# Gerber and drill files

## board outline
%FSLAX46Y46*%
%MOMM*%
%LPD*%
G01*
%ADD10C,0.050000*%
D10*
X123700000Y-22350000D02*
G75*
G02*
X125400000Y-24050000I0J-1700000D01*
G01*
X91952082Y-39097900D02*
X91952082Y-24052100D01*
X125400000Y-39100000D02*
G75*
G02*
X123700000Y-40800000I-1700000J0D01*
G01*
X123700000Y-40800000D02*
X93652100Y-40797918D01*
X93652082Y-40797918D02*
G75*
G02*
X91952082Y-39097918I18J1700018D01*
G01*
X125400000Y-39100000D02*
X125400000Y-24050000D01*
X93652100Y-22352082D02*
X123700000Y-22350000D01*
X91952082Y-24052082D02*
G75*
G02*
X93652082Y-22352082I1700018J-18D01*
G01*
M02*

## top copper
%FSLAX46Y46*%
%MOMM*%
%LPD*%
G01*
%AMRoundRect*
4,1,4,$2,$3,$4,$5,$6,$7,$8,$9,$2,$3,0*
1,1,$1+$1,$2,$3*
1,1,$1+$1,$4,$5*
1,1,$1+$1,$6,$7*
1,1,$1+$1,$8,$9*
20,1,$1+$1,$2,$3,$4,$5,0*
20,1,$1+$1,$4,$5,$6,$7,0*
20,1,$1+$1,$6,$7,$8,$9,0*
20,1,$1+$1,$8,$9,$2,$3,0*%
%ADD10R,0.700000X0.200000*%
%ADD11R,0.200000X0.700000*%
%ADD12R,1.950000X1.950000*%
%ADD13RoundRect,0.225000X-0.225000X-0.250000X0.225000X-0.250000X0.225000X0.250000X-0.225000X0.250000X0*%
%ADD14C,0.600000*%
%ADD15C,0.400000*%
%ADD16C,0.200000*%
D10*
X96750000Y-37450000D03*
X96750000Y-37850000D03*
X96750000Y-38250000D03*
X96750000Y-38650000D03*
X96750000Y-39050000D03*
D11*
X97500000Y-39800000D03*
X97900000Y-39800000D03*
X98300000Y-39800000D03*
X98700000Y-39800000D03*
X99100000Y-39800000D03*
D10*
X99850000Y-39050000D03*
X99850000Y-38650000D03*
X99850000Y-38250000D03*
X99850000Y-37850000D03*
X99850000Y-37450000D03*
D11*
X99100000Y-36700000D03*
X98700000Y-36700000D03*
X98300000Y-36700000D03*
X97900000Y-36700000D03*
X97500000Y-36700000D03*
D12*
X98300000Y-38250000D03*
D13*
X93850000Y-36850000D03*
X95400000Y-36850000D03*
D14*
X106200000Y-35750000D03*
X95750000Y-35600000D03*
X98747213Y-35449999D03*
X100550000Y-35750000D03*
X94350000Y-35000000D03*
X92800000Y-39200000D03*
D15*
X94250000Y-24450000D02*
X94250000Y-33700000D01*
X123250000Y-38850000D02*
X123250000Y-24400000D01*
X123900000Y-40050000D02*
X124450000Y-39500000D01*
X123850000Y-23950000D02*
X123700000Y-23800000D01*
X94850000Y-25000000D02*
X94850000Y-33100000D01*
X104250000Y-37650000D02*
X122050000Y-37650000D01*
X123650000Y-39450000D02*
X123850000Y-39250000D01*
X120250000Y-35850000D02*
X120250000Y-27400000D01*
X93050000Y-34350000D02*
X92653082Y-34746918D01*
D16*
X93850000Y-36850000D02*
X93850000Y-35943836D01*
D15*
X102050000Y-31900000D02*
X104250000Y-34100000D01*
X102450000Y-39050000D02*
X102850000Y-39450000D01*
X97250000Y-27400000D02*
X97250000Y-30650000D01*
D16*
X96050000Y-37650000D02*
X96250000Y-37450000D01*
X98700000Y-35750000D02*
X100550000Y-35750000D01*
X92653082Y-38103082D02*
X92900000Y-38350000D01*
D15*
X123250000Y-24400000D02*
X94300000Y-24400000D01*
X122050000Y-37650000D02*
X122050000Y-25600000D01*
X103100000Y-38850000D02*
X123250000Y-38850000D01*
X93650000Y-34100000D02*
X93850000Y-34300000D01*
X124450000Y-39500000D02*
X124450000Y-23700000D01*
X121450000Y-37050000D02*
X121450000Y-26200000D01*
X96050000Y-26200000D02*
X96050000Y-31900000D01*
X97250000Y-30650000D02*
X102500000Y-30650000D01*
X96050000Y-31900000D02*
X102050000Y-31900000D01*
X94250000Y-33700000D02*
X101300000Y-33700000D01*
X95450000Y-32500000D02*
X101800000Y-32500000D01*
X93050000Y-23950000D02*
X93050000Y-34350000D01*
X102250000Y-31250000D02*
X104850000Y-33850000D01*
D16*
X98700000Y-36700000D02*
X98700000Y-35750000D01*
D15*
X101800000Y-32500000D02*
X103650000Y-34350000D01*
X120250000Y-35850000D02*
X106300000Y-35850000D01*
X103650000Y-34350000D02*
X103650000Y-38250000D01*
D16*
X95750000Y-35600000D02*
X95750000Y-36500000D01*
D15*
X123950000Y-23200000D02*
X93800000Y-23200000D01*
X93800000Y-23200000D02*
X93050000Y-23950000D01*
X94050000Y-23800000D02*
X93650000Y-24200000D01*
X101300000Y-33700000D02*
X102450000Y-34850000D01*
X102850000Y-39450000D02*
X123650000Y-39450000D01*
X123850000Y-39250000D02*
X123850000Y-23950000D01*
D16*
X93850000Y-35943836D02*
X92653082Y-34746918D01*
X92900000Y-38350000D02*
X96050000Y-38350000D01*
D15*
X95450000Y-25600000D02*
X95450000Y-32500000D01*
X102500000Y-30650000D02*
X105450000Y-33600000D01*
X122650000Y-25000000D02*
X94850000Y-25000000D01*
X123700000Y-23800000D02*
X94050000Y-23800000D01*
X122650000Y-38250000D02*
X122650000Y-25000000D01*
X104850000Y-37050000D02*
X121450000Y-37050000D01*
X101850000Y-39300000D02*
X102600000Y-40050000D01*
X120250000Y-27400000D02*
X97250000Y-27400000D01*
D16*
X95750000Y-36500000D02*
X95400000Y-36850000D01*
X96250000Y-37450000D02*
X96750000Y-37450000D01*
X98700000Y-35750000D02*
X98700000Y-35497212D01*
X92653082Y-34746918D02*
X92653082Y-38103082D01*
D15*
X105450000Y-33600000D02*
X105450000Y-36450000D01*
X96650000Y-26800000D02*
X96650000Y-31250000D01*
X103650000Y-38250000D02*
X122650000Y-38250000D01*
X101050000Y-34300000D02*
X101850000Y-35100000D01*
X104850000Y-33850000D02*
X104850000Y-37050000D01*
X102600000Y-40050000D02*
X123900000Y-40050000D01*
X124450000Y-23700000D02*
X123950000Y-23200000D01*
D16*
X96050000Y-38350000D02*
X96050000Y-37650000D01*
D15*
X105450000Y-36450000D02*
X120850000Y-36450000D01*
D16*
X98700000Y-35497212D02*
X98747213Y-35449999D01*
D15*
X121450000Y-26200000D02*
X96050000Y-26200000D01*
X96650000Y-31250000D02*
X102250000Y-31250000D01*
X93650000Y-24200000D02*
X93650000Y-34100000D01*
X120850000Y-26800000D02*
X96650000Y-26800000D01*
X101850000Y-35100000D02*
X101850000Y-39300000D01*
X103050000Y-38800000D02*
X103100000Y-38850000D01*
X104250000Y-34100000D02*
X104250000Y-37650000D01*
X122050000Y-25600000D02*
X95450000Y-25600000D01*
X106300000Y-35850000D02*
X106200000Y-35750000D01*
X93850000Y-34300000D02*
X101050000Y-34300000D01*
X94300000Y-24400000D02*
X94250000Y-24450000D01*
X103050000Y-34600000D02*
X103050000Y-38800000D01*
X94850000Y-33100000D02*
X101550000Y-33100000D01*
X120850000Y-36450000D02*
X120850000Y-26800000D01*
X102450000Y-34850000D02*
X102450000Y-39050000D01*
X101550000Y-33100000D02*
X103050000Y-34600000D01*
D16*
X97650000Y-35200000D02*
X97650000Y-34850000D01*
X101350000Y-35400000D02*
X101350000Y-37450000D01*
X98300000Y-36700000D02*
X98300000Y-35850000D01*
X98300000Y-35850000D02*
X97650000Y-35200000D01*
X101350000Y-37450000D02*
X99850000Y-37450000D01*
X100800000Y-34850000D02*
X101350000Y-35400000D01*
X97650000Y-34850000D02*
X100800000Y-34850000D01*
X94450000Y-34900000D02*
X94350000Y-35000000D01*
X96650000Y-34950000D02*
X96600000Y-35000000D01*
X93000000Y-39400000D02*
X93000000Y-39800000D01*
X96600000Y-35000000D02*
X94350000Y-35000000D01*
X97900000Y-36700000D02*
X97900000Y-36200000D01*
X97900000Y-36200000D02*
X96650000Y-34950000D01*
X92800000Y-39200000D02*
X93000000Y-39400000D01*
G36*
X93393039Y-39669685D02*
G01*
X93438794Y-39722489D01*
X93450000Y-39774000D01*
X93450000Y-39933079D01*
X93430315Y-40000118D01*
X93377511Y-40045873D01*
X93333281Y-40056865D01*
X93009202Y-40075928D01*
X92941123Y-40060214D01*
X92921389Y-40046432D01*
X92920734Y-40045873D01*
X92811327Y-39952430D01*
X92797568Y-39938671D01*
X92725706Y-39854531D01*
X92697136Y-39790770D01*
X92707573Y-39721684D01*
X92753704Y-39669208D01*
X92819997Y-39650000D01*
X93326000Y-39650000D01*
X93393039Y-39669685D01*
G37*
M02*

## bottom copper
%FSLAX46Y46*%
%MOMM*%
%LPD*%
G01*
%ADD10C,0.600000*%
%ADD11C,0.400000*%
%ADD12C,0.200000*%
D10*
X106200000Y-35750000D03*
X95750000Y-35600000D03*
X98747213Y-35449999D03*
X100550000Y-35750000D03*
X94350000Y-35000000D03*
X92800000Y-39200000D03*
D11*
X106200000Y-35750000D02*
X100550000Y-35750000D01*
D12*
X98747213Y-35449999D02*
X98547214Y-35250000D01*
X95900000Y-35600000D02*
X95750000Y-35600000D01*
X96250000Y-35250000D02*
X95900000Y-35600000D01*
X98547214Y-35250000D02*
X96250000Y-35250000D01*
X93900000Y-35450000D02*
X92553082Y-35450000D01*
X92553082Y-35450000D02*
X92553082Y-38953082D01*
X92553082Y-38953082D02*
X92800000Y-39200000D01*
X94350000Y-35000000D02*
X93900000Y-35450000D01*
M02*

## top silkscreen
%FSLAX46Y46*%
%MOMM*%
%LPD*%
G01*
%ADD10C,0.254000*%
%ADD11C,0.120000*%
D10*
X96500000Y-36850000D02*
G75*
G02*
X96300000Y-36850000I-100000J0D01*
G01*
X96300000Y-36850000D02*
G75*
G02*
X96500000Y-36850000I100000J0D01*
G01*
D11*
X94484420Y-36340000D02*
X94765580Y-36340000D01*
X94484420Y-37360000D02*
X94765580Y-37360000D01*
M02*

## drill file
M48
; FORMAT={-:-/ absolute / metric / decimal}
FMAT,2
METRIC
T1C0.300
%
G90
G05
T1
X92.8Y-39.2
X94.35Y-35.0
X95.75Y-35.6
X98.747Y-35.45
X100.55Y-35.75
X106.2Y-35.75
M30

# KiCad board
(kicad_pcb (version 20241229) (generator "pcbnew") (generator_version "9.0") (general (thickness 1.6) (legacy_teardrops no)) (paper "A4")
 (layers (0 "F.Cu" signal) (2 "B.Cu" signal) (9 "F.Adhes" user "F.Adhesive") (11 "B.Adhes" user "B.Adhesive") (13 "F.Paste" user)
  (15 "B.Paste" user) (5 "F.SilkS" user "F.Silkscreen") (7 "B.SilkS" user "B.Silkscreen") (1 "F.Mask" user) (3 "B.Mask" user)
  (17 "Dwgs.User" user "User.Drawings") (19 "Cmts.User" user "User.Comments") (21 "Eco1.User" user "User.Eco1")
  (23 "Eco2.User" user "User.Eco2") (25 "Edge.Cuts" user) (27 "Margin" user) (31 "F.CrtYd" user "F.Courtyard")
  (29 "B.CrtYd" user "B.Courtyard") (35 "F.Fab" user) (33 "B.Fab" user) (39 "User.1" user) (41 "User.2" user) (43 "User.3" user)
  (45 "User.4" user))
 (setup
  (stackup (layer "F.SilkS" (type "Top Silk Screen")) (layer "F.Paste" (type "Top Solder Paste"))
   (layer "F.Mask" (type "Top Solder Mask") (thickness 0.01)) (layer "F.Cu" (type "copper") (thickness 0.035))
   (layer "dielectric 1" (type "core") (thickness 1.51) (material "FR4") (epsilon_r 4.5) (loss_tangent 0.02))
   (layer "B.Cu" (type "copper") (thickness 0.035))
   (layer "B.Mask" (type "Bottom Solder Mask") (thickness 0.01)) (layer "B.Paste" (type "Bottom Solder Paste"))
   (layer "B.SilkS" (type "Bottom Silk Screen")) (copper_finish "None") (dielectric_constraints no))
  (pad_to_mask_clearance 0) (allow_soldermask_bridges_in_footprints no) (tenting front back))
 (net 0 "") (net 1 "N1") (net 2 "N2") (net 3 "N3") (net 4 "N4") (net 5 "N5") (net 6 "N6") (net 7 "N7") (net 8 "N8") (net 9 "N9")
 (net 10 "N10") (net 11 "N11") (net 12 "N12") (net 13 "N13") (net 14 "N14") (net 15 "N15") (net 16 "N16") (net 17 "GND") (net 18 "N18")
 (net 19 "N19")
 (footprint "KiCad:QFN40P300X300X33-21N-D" (layer "F.Cu") (at 98.3 38.25)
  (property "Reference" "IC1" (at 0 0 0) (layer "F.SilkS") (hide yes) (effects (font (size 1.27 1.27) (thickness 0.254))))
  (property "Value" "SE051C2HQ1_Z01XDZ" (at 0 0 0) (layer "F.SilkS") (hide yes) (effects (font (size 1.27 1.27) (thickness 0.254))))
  (fp_circle (center -1.9 -1.4) (end -1.8 -1.4) (stroke (width 0.254) (type solid)) (fill no) (layer "F.SilkS"))
  (pad "1" smd rect (at -1.55 -0.8 90) (size 0.2 0.7) (layers "F.Cu" "F.Mask" "F.Paste") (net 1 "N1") (solder_mask_margin 0.04)
   (thermal_bridge_angle 45))
  (pad "2" smd rect (at -1.55 -0.4 90) (size 0.2 0.7) (layers "F.Cu" "F.Mask" "F.Paste") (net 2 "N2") (solder_mask_margin 0.04)
   (thermal_bridge_angle 45))
  (pad "3" smd rect (at -1.55 0 90) (size 0.2 0.7) (layers "F.Cu" "F.Mask" "F.Paste") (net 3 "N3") (solder_mask_margin 0.04)
   (thermal_bridge_angle 45))
  (pad "4" smd rect (at -1.55 0.4 90) (size 0.2 0.7) (layers "F.Cu" "F.Mask" "F.Paste") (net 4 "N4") (solder_mask_margin 0.04)
   (thermal_bridge_angle 45))
  (pad "5" smd rect (at -1.55 0.8 90) (size 0.2 0.7) (layers "F.Cu" "F.Mask" "F.Paste") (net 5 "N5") (solder_mask_margin 0.04)
   (thermal_bridge_angle 45))
  (pad "6" smd rect (at -0.8 1.55) (size 0.2 0.7) (layers "F.Cu" "F.Mask" "F.Paste") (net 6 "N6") (solder_mask_margin 0.04)
   (thermal_bridge_angle 45))
  (pad "7" smd rect (at -0.4 1.55) (size 0.2 0.7) (layers "F.Cu" "F.Mask" "F.Paste") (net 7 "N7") (solder_mask_margin 0.04)
   (thermal_bridge_angle 45))
  (pad "8" smd rect (at 0 1.55) (size 0.2 0.7) (layers "F.Cu" "F.Mask" "F.Paste") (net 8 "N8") (solder_mask_margin 0.04)
   (thermal_bridge_angle 45))
  (pad "9" smd rect (at 0.4 1.55) (size 0.2 0.7) (layers "F.Cu" "F.Mask" "F.Paste") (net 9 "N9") (solder_mask_margin 0.04)
   (thermal_bridge_angle 45))
  (pad "10" smd rect (at 0.8 1.55) (size 0.2 0.7) (layers "F.Cu" "F.Mask" "F.Paste") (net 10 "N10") (solder_mask_margin 0.04)
   (thermal_bridge_angle 45))
  (pad "11" smd rect (at 1.55 0.8 90) (size 0.2 0.7) (layers "F.Cu" "F.Mask" "F.Paste") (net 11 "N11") (solder_mask_margin 0.04)
   (thermal_bridge_angle 45))
  (pad "12" smd rect (at 1.55 0.4 90) (size 0.2 0.7) (layers "F.Cu" "F.Mask" "F.Paste") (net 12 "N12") (solder_mask_margin 0.04)
   (thermal_bridge_angle 45))
  (pad "13" smd rect (at 1.55 0 90) (size 0.2 0.7) (layers "F.Cu" "F.Mask" "F.Paste") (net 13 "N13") (solder_mask_margin 0.04)
   (thermal_bridge_angle 45))
  (pad "14" smd rect (at 1.55 -0.4 90) (size 0.2 0.7) (layers "F.Cu" "F.Mask" "F.Paste") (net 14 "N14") (solder_mask_margin 0.04)
   (thermal_bridge_angle 45))
  (pad "15" smd rect (at 1.55 -0.8 90) (size 0.2 0.7) (layers "F.Cu" "F.Mask" "F.Paste") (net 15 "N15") (solder_mask_margin 0.04)
   (thermal_bridge_angle 45))
  (pad "16" smd rect (at 0.8 -1.55) (size 0.2 0.7) (layers "F.Cu" "F.Mask" "F.Paste") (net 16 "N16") (solder_mask_margin 0.04)
   (thermal_bridge_angle 45))
  (pad "17" smd rect (at 0.4 -1.55) (size 0.2 0.7) (layers "F.Cu" "F.Mask" "F.Paste") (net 1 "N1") (solder_mask_margin 0.04)
   (thermal_bridge_angle 45))
  (pad "18" smd rect (at 0 -1.55) (size 0.2 0.7) (layers "F.Cu" "F.Mask" "F.Paste") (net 15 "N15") (solder_mask_margin 0.04)
   (thermal_bridge_angle 45))
  (pad "19" smd rect (at -0.4 -1.55) (size 0.2 0.7) (layers "F.Cu" "F.Mask" "F.Paste") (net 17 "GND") (solder_mask_margin 0.04)
   (thermal_bridge_angle 45))
  (pad "20" smd rect (at -0.8 -1.55) (size 0.2 0.7) (layers "F.Cu" "F.Mask" "F.Paste") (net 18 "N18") (solder_mask_margin 0.04)
   (thermal_bridge_angle 45))
  (pad "21" smd rect (at 0 0) (size 1.95 1.95) (layers "F.Cu" "F.Mask" "F.Paste") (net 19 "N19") (thermal_bridge_angle 45)))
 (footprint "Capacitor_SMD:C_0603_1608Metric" (layer "F.Cu") (at 94.625 36.85)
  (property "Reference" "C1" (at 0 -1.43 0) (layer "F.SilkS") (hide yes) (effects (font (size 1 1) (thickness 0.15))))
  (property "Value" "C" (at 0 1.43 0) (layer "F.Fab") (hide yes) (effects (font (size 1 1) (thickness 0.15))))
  (fp_line (start -0.14058 -0.51) (end 0.14058 -0.51) (stroke (width 0.12) (type solid)) (layer "F.SilkS"))
  (fp_line (start -0.14058 0.51) (end 0.14058 0.51) (stroke (width 0.12) (type solid)) (layer "F.SilkS"))
  (pad "1" smd roundrect (at -0.775 0) (size 0.9 0.95) (layers "F.Cu" "F.Mask" "F.Paste") (roundrect_rratio 0.25) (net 1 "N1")
   (solder_mask_margin 0.04))
  (pad "2" smd roundrect (at 0.775 0) (size 0.9 0.95) (layers "F.Cu" "F.Mask" "F.Paste") (roundrect_rratio 0.25) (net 1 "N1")
   (solder_mask_margin 0.04)))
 (gr_arc (start 123.7 22.35) (mid 124.902082 22.847918) (end 125.4 24.05) (stroke (width 0.05) (type default)) (layer "Edge.Cuts"))
 (gr_line (start 91.952082 39.0979) (end 91.952082 24.0521) (stroke (width 0.05) (type default)) (layer "Edge.Cuts"))
 (gr_arc (start 125.4 39.1) (mid 124.902082 40.302082) (end 123.7 40.8) (stroke (width 0.05) (type default)) (layer "Edge.Cuts"))
 (gr_line (start 123.7 40.8) (end 93.6521 40.797918) (stroke (width 0.05) (type default)) (layer "Edge.Cuts"))
 (gr_arc (start 93.652082 40.797918) (mid 92.45 40.3) (end 91.952082 39.097918) (stroke (width 0.05) (type default)) (layer "Edge.Cuts"))
 (gr_line (start 125.4 39.1) (end 125.4 24.05) (stroke (width 0.05) (type default)) (layer "Edge.Cuts"))
 (gr_line (start 93.6521 22.352082) (end 123.7 22.35) (stroke (width 0.05) (type default)) (layer "Edge.Cuts"))
 (gr_arc (start 91.952082 24.052082) (mid 92.45 22.85) (end 93.652082 22.352082) (stroke (width 0.05) (type default)) (layer "Edge.Cuts"))
 (segment (start 94.25 24.45) (end 94.25 33.7) (width 0.4) (layer "F.Cu") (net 1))
 (segment (start 123.25 38.85) (end 123.25 24.4) (width 0.4) (layer "F.Cu") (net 1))
 (segment (start 123.9 40.05) (end 124.45 39.5) (width 0.4) (layer "F.Cu") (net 1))
 (segment (start 123.85 23.95) (end 123.7 23.8) (width 0.4) (layer "F.Cu") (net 1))
 (segment (start 94.85 25) (end 94.85 33.1) (width 0.4) (layer "F.Cu") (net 1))
 (segment (start 104.25 37.65) (end 122.05 37.65) (width 0.4) (layer "F.Cu") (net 1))
 (segment (start 123.65 39.45) (end 123.85 39.25) (width 0.4) (layer "F.Cu") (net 1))
 (segment (start 120.25 35.85) (end 120.25 27.4) (width 0.4) (layer "F.Cu") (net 1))
 (segment (start 93.05 34.35) (end 92.653082 34.746918) (width 0.4) (layer "F.Cu") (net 1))
 (segment (start 93.85 36.85) (end 93.85 35.943836) (width 0.2) (layer "F.Cu") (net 1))
 (segment (start 102.05 31.9) (end 104.25 34.1) (width 0.4) (layer "F.Cu") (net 1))
 (segment (start 102.45 39.05) (end 102.85 39.45) (width 0.4) (layer "F.Cu") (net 1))
 (segment (start 97.25 27.4) (end 97.25 30.65) (width 0.4) (layer "F.Cu") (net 1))
 (segment (start 96.05 37.65) (end 96.25 37.45) (width 0.2) (layer "F.Cu") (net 1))
 (segment (start 98.7 35.75) (end 100.55 35.75) (width 0.2) (layer "F.Cu") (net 1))
 (segment (start 92.653082 38.103082) (end 92.9 38.35) (width 0.2) (layer "F.Cu") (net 1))
 (segment (start 123.25 24.4) (end 94.3 24.4) (width 0.4) (layer "F.Cu") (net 1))
 (segment (start 122.05 37.65) (end 122.05 25.6) (width 0.4) (layer "F.Cu") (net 1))
 (segment (start 103.1 38.85) (end 123.25 38.85) (width 0.4) (layer "F.Cu") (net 1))
 (segment (start 93.65 34.1) (end 93.85 34.3) (width 0.4) (layer "F.Cu") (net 1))
 (segment (start 124.45 39.5) (end 124.45 23.7) (width 0.4) (layer "F.Cu") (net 1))
 (segment (start 121.45 37.05) (end 121.45 26.2) (width 0.4) (layer "F.Cu") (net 1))
 (segment (start 96.05 26.2) (end 96.05 31.9) (width 0.4) (layer "F.Cu") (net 1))
 (segment (start 97.25 30.65) (end 102.5 30.65) (width 0.4) (layer "F.Cu") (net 1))
 (segment (start 96.05 31.9) (end 102.05 31.9) (width 0.4) (layer "F.Cu") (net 1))
 (segment (start 94.25 33.7) (end 101.3 33.7) (width 0.4) (layer "F.Cu") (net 1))
 (segment (start 95.45 32.5) (end 101.8 32.5) (width 0.4) (layer "F.Cu") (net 1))
 (segment (start 93.05 23.95) (end 93.05 34.35) (width 0.4) (layer "F.Cu") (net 1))
 (segment (start 102.25 31.25) (end 104.85 33.85) (width 0.4) (layer "F.Cu") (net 1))
 (segment (start 98.7 36.7) (end 98.7 35.75) (width 0.2) (layer "F.Cu") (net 1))
 (segment (start 101.8 32.5) (end 103.65 34.35) (width 0.4) (layer "F.Cu") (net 1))
 (segment (start 120.25 35.85) (end 106.3 35.85) (width 0.4) (layer "F.Cu") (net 1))
 (segment (start 103.65 34.35) (end 103.65 38.25) (width 0.4) (layer "F.Cu") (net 1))
 (segment (start 95.75 35.6) (end 95.75 36.5) (width 0.2) (layer "F.Cu") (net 1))
 (segment (start 123.95 23.2) (end 93.8 23.2) (width 0.4) (layer "F.Cu") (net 1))
 (segment (start 93.8 23.2) (end 93.05 23.95) (width 0.4) (layer "F.Cu") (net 1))
 (segment (start 94.05 23.8) (end 93.65 24.2) (width 0.4) (layer "F.Cu") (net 1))
 (segment (start 101.3 33.7) (end 102.45 34.85) (width 0.4) (layer "F.Cu") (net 1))
 (segment (start 102.85 39.45) (end 123.65 39.45) (width 0.4) (layer "F.Cu") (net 1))
 (segment (start 123.85 39.25) (end 123.85 23.95) (width 0.4) (layer "F.Cu") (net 1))
 (segment (start 93.85 35.943836) (end 92.653082 34.746918) (width 0.2) (layer "F.Cu") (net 1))
 (segment (start 92.9 38.35) (end 96.05 38.35) (width 0.2) (layer "F.Cu") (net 1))
 (segment (start 95.45 25.6) (end 95.45 32.5) (width 0.4) (layer "F.Cu") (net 1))
 (segment (start 102.5 30.65) (end 105.45 33.6) (width 0.4) (layer "F.Cu") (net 1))
 (segment (start 122.65 25) (end 94.85 25) (width 0.4) (layer "F.Cu") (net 1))
 (segment (start 123.7 23.8) (end 94.05 23.8) (width 0.4) (layer "F.Cu") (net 1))
 (segment (start 122.65 38.25) (end 122.65 25) (width 0.4) (layer "F.Cu") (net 1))
 (segment (start 104.85 37.05) (end 121.45 37.05) (width 0.4) (layer "F.Cu") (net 1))
 (segment (start 101.85 39.3) (end 102.6 40.05) (width 0.4) (layer "F.Cu") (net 1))
 (segment (start 120.25 27.4) (end 97.25 27.4) (width 0.4) (layer "F.Cu") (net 1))
 (segment (start 95.75 36.5) (end 95.4 36.85) (width 0.2) (layer "F.Cu") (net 1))
 (segment (start 96.25 37.45) (end 96.75 37.45) (width 0.2) (layer "F.Cu") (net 1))
 (segment (start 98.7 35.75) (end 98.7 35.497212) (width 0.2) (layer "F.Cu") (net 1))
 (segment (start 92.653082 34.746918) (end 92.653082 38.103082) (width 0.2) (layer "F.Cu") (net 1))
 (segment (start 105.45 33.6) (end 105.45 36.45) (width 0.4) (layer "F.Cu") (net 1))
 (segment (start 96.65 26.8) (end 96.65 31.25) (width 0.4) (layer "F.Cu") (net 1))
 (segment (start 103.65 38.25) (end 122.65 38.25) (width 0.4) (layer "F.Cu") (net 1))
 (segment (start 101.05 34.3) (end 101.85 35.1) (width 0.4) (layer "F.Cu") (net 1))
 (segment (start 104.85 33.85) (end 104.85 37.05) (width 0.4) (layer "F.Cu") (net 1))
 (segment (start 102.6 40.05) (end 123.9 40.05) (width 0.4) (layer "F.Cu") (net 1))
 (segment (start 124.45 23.7) (end 123.95 23.2) (width 0.4) (layer "F.Cu") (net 1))
 (segment (start 96.05 38.35) (end 96.05 37.65) (width 0.2) (layer "F.Cu") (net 1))
 (segment (start 105.45 36.45) (end 120.85 36.45) (width 0.4) (layer "F.Cu") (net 1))
 (segment (start 98.7 35.497212) (end 98.747213 35.449999) (width 0.2) (layer "F.Cu") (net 1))
 (segment (start 121.45 26.2) (end 96.05 26.2) (width 0.4) (layer "F.Cu") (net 1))
 (segment (start 96.65 31.25) (end 102.25 31.25) (width 0.4) (layer "F.Cu") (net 1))
 (segment (start 93.65 24.2) (end 93.65 34.1) (width 0.4) (layer "F.Cu") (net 1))
 (segment (start 120.85 26.8) (end 96.65 26.8) (width 0.4) (layer "F.Cu") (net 1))
 (segment (start 101.85 35.1) (end 101.85 39.3) (width 0.4) (layer "F.Cu") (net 1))
 (segment (start 103.05 38.8) (end 103.1 38.85) (width 0.4) (layer "F.Cu") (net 1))
 (segment (start 104.25 34.1) (end 104.25 37.65) (width 0.4) (layer "F.Cu") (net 1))
 (segment (start 122.05 25.6) (end 95.45 25.6) (width 0.4) (layer "F.Cu") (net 1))
 (segment (start 106.3 35.85) (end 106.2 35.75) (width 0.4) (layer "F.Cu") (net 1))
 (segment (start 93.85 34.3) (end 101.05 34.3) (width 0.4) (layer "F.Cu") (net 1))
 (segment (start 94.3 24.4) (end 94.25 24.45) (width 0.4) (layer "F.Cu") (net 1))
 (segment (start 103.05 34.6) (end 103.05 38.8) (width 0.4) (layer "F.Cu") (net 1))
 (segment (start 94.85 33.1) (end 101.55 33.1) (width 0.4) (layer "F.Cu") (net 1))
 (segment (start 120.85 36.45) (end 120.85 26.8) (width 0.4) (layer "F.Cu") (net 1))
 (segment (start 102.45 34.85) (end 102.45 39.05) (width 0.4) (layer "F.Cu") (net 1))
 (segment (start 101.55 33.1) (end 103.05 34.6) (width 0.4) (layer "F.Cu") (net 1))
 (via (at 106.2 35.75) (size 0.6) (drill 0.3) (layers "F.Cu" "B.Cu") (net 1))
 (via (at 95.75 35.6) (size 0.6) (drill 0.3) (layers "F.Cu" "B.Cu") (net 1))
 (via (at 98.747213 35.449999) (size 0.6) (drill 0.3) (layers "F.Cu" "B.Cu") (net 1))
 (via (at 100.55 35.75) (size 0.6) (drill 0.3) (layers "F.Cu" "B.Cu") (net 1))
 (segment (start 106.2 35.75) (end 100.55 35.75) (width 0.4) (layer "B.Cu") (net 1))
 (segment (start 98.747213 35.449999) (end 98.547214 35.25) (width 0.2) (layer "B.Cu") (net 1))
 (segment (start 95.9 35.6) (end 95.75 35.6) (width 0.2) (layer "B.Cu") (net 1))
 (segment (start 96.25 35.25) (end 95.9 35.6) (width 0.2) (layer "B.Cu") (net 1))
 (segment (start 98.547214 35.25) (end 96.25 35.25) (width 0.2) (layer "B.Cu") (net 1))
 (segment (start 97.65 35.2) (end 97.65 34.85) (width 0.2) (layer "F.Cu") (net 15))
 (segment (start 101.35 35.4) (end 101.35 37.45) (width 0.2) (layer "F.Cu") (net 15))
 (segment (start 98.3 36.7) (end 98.3 35.85) (width 0.2) (layer "F.Cu") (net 15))
 (segment (start 98.3 35.85) (end 97.65 35.2) (width 0.2) (layer "F.Cu") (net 15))
 (segment (start 101.35 37.45) (end 99.85 37.45) (width 0.2) (layer "F.Cu") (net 15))
 (segment (start 100.8 34.85) (end 101.35 35.4) (width 0.2) (layer "F.Cu") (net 15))
 (segment (start 97.65 34.85) (end 100.8 34.85) (width 0.2) (layer "F.Cu") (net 15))
 (segment (start 94.45 34.9) (end 94.35 35) (width 0.2) (layer "F.Cu") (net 17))
 (segment (start 96.65 34.95) (end 96.6 35) (width 0.2) (layer "F.Cu") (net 17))
 (segment (start 93 39.4) (end 93 39.8) (width 0.2) (layer "F.Cu") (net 17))
 (segment (start 96.6 35) (end 94.35 35) (width 0.2) (layer "F.Cu") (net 17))
 (segment (start 97.9 36.7) (end 97.9 36.2) (width 0.2) (layer "F.Cu") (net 17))
 (segment (start 97.9 36.2) (end 96.65 34.95) (width 0.2) (layer "F.Cu") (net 17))
 (segment (start 92.8 39.2) (end 93 39.4) (width 0.2) (layer "F.Cu") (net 17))
 (via (at 94.35 35) (size 0.6) (drill 0.3) (layers "F.Cu" "B.Cu") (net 17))
 (via (at 92.8 39.2) (size 0.6) (drill 0.3) (layers "F.Cu" "B.Cu") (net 17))
 (segment (start 93.9 35.45) (end 92.553082 35.45) (width 0.2) (layer "B.Cu") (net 17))
 (segment (start 92.553082 35.45) (end 92.553082 38.953082) (width 0.2) (layer "B.Cu") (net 17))
 (segment (start 92.553082 38.953082) (end 92.8 39.2) (width 0.2) (layer "B.Cu") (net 17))
 (segment (start 94.35 35) (end 93.9 35.45) (width 0.2) (layer "B.Cu") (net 17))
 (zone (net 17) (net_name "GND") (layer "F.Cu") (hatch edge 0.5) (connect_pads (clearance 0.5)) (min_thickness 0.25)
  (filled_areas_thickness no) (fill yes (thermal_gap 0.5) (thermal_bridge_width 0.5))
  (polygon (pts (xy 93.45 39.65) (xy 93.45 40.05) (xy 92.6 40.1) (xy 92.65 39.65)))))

